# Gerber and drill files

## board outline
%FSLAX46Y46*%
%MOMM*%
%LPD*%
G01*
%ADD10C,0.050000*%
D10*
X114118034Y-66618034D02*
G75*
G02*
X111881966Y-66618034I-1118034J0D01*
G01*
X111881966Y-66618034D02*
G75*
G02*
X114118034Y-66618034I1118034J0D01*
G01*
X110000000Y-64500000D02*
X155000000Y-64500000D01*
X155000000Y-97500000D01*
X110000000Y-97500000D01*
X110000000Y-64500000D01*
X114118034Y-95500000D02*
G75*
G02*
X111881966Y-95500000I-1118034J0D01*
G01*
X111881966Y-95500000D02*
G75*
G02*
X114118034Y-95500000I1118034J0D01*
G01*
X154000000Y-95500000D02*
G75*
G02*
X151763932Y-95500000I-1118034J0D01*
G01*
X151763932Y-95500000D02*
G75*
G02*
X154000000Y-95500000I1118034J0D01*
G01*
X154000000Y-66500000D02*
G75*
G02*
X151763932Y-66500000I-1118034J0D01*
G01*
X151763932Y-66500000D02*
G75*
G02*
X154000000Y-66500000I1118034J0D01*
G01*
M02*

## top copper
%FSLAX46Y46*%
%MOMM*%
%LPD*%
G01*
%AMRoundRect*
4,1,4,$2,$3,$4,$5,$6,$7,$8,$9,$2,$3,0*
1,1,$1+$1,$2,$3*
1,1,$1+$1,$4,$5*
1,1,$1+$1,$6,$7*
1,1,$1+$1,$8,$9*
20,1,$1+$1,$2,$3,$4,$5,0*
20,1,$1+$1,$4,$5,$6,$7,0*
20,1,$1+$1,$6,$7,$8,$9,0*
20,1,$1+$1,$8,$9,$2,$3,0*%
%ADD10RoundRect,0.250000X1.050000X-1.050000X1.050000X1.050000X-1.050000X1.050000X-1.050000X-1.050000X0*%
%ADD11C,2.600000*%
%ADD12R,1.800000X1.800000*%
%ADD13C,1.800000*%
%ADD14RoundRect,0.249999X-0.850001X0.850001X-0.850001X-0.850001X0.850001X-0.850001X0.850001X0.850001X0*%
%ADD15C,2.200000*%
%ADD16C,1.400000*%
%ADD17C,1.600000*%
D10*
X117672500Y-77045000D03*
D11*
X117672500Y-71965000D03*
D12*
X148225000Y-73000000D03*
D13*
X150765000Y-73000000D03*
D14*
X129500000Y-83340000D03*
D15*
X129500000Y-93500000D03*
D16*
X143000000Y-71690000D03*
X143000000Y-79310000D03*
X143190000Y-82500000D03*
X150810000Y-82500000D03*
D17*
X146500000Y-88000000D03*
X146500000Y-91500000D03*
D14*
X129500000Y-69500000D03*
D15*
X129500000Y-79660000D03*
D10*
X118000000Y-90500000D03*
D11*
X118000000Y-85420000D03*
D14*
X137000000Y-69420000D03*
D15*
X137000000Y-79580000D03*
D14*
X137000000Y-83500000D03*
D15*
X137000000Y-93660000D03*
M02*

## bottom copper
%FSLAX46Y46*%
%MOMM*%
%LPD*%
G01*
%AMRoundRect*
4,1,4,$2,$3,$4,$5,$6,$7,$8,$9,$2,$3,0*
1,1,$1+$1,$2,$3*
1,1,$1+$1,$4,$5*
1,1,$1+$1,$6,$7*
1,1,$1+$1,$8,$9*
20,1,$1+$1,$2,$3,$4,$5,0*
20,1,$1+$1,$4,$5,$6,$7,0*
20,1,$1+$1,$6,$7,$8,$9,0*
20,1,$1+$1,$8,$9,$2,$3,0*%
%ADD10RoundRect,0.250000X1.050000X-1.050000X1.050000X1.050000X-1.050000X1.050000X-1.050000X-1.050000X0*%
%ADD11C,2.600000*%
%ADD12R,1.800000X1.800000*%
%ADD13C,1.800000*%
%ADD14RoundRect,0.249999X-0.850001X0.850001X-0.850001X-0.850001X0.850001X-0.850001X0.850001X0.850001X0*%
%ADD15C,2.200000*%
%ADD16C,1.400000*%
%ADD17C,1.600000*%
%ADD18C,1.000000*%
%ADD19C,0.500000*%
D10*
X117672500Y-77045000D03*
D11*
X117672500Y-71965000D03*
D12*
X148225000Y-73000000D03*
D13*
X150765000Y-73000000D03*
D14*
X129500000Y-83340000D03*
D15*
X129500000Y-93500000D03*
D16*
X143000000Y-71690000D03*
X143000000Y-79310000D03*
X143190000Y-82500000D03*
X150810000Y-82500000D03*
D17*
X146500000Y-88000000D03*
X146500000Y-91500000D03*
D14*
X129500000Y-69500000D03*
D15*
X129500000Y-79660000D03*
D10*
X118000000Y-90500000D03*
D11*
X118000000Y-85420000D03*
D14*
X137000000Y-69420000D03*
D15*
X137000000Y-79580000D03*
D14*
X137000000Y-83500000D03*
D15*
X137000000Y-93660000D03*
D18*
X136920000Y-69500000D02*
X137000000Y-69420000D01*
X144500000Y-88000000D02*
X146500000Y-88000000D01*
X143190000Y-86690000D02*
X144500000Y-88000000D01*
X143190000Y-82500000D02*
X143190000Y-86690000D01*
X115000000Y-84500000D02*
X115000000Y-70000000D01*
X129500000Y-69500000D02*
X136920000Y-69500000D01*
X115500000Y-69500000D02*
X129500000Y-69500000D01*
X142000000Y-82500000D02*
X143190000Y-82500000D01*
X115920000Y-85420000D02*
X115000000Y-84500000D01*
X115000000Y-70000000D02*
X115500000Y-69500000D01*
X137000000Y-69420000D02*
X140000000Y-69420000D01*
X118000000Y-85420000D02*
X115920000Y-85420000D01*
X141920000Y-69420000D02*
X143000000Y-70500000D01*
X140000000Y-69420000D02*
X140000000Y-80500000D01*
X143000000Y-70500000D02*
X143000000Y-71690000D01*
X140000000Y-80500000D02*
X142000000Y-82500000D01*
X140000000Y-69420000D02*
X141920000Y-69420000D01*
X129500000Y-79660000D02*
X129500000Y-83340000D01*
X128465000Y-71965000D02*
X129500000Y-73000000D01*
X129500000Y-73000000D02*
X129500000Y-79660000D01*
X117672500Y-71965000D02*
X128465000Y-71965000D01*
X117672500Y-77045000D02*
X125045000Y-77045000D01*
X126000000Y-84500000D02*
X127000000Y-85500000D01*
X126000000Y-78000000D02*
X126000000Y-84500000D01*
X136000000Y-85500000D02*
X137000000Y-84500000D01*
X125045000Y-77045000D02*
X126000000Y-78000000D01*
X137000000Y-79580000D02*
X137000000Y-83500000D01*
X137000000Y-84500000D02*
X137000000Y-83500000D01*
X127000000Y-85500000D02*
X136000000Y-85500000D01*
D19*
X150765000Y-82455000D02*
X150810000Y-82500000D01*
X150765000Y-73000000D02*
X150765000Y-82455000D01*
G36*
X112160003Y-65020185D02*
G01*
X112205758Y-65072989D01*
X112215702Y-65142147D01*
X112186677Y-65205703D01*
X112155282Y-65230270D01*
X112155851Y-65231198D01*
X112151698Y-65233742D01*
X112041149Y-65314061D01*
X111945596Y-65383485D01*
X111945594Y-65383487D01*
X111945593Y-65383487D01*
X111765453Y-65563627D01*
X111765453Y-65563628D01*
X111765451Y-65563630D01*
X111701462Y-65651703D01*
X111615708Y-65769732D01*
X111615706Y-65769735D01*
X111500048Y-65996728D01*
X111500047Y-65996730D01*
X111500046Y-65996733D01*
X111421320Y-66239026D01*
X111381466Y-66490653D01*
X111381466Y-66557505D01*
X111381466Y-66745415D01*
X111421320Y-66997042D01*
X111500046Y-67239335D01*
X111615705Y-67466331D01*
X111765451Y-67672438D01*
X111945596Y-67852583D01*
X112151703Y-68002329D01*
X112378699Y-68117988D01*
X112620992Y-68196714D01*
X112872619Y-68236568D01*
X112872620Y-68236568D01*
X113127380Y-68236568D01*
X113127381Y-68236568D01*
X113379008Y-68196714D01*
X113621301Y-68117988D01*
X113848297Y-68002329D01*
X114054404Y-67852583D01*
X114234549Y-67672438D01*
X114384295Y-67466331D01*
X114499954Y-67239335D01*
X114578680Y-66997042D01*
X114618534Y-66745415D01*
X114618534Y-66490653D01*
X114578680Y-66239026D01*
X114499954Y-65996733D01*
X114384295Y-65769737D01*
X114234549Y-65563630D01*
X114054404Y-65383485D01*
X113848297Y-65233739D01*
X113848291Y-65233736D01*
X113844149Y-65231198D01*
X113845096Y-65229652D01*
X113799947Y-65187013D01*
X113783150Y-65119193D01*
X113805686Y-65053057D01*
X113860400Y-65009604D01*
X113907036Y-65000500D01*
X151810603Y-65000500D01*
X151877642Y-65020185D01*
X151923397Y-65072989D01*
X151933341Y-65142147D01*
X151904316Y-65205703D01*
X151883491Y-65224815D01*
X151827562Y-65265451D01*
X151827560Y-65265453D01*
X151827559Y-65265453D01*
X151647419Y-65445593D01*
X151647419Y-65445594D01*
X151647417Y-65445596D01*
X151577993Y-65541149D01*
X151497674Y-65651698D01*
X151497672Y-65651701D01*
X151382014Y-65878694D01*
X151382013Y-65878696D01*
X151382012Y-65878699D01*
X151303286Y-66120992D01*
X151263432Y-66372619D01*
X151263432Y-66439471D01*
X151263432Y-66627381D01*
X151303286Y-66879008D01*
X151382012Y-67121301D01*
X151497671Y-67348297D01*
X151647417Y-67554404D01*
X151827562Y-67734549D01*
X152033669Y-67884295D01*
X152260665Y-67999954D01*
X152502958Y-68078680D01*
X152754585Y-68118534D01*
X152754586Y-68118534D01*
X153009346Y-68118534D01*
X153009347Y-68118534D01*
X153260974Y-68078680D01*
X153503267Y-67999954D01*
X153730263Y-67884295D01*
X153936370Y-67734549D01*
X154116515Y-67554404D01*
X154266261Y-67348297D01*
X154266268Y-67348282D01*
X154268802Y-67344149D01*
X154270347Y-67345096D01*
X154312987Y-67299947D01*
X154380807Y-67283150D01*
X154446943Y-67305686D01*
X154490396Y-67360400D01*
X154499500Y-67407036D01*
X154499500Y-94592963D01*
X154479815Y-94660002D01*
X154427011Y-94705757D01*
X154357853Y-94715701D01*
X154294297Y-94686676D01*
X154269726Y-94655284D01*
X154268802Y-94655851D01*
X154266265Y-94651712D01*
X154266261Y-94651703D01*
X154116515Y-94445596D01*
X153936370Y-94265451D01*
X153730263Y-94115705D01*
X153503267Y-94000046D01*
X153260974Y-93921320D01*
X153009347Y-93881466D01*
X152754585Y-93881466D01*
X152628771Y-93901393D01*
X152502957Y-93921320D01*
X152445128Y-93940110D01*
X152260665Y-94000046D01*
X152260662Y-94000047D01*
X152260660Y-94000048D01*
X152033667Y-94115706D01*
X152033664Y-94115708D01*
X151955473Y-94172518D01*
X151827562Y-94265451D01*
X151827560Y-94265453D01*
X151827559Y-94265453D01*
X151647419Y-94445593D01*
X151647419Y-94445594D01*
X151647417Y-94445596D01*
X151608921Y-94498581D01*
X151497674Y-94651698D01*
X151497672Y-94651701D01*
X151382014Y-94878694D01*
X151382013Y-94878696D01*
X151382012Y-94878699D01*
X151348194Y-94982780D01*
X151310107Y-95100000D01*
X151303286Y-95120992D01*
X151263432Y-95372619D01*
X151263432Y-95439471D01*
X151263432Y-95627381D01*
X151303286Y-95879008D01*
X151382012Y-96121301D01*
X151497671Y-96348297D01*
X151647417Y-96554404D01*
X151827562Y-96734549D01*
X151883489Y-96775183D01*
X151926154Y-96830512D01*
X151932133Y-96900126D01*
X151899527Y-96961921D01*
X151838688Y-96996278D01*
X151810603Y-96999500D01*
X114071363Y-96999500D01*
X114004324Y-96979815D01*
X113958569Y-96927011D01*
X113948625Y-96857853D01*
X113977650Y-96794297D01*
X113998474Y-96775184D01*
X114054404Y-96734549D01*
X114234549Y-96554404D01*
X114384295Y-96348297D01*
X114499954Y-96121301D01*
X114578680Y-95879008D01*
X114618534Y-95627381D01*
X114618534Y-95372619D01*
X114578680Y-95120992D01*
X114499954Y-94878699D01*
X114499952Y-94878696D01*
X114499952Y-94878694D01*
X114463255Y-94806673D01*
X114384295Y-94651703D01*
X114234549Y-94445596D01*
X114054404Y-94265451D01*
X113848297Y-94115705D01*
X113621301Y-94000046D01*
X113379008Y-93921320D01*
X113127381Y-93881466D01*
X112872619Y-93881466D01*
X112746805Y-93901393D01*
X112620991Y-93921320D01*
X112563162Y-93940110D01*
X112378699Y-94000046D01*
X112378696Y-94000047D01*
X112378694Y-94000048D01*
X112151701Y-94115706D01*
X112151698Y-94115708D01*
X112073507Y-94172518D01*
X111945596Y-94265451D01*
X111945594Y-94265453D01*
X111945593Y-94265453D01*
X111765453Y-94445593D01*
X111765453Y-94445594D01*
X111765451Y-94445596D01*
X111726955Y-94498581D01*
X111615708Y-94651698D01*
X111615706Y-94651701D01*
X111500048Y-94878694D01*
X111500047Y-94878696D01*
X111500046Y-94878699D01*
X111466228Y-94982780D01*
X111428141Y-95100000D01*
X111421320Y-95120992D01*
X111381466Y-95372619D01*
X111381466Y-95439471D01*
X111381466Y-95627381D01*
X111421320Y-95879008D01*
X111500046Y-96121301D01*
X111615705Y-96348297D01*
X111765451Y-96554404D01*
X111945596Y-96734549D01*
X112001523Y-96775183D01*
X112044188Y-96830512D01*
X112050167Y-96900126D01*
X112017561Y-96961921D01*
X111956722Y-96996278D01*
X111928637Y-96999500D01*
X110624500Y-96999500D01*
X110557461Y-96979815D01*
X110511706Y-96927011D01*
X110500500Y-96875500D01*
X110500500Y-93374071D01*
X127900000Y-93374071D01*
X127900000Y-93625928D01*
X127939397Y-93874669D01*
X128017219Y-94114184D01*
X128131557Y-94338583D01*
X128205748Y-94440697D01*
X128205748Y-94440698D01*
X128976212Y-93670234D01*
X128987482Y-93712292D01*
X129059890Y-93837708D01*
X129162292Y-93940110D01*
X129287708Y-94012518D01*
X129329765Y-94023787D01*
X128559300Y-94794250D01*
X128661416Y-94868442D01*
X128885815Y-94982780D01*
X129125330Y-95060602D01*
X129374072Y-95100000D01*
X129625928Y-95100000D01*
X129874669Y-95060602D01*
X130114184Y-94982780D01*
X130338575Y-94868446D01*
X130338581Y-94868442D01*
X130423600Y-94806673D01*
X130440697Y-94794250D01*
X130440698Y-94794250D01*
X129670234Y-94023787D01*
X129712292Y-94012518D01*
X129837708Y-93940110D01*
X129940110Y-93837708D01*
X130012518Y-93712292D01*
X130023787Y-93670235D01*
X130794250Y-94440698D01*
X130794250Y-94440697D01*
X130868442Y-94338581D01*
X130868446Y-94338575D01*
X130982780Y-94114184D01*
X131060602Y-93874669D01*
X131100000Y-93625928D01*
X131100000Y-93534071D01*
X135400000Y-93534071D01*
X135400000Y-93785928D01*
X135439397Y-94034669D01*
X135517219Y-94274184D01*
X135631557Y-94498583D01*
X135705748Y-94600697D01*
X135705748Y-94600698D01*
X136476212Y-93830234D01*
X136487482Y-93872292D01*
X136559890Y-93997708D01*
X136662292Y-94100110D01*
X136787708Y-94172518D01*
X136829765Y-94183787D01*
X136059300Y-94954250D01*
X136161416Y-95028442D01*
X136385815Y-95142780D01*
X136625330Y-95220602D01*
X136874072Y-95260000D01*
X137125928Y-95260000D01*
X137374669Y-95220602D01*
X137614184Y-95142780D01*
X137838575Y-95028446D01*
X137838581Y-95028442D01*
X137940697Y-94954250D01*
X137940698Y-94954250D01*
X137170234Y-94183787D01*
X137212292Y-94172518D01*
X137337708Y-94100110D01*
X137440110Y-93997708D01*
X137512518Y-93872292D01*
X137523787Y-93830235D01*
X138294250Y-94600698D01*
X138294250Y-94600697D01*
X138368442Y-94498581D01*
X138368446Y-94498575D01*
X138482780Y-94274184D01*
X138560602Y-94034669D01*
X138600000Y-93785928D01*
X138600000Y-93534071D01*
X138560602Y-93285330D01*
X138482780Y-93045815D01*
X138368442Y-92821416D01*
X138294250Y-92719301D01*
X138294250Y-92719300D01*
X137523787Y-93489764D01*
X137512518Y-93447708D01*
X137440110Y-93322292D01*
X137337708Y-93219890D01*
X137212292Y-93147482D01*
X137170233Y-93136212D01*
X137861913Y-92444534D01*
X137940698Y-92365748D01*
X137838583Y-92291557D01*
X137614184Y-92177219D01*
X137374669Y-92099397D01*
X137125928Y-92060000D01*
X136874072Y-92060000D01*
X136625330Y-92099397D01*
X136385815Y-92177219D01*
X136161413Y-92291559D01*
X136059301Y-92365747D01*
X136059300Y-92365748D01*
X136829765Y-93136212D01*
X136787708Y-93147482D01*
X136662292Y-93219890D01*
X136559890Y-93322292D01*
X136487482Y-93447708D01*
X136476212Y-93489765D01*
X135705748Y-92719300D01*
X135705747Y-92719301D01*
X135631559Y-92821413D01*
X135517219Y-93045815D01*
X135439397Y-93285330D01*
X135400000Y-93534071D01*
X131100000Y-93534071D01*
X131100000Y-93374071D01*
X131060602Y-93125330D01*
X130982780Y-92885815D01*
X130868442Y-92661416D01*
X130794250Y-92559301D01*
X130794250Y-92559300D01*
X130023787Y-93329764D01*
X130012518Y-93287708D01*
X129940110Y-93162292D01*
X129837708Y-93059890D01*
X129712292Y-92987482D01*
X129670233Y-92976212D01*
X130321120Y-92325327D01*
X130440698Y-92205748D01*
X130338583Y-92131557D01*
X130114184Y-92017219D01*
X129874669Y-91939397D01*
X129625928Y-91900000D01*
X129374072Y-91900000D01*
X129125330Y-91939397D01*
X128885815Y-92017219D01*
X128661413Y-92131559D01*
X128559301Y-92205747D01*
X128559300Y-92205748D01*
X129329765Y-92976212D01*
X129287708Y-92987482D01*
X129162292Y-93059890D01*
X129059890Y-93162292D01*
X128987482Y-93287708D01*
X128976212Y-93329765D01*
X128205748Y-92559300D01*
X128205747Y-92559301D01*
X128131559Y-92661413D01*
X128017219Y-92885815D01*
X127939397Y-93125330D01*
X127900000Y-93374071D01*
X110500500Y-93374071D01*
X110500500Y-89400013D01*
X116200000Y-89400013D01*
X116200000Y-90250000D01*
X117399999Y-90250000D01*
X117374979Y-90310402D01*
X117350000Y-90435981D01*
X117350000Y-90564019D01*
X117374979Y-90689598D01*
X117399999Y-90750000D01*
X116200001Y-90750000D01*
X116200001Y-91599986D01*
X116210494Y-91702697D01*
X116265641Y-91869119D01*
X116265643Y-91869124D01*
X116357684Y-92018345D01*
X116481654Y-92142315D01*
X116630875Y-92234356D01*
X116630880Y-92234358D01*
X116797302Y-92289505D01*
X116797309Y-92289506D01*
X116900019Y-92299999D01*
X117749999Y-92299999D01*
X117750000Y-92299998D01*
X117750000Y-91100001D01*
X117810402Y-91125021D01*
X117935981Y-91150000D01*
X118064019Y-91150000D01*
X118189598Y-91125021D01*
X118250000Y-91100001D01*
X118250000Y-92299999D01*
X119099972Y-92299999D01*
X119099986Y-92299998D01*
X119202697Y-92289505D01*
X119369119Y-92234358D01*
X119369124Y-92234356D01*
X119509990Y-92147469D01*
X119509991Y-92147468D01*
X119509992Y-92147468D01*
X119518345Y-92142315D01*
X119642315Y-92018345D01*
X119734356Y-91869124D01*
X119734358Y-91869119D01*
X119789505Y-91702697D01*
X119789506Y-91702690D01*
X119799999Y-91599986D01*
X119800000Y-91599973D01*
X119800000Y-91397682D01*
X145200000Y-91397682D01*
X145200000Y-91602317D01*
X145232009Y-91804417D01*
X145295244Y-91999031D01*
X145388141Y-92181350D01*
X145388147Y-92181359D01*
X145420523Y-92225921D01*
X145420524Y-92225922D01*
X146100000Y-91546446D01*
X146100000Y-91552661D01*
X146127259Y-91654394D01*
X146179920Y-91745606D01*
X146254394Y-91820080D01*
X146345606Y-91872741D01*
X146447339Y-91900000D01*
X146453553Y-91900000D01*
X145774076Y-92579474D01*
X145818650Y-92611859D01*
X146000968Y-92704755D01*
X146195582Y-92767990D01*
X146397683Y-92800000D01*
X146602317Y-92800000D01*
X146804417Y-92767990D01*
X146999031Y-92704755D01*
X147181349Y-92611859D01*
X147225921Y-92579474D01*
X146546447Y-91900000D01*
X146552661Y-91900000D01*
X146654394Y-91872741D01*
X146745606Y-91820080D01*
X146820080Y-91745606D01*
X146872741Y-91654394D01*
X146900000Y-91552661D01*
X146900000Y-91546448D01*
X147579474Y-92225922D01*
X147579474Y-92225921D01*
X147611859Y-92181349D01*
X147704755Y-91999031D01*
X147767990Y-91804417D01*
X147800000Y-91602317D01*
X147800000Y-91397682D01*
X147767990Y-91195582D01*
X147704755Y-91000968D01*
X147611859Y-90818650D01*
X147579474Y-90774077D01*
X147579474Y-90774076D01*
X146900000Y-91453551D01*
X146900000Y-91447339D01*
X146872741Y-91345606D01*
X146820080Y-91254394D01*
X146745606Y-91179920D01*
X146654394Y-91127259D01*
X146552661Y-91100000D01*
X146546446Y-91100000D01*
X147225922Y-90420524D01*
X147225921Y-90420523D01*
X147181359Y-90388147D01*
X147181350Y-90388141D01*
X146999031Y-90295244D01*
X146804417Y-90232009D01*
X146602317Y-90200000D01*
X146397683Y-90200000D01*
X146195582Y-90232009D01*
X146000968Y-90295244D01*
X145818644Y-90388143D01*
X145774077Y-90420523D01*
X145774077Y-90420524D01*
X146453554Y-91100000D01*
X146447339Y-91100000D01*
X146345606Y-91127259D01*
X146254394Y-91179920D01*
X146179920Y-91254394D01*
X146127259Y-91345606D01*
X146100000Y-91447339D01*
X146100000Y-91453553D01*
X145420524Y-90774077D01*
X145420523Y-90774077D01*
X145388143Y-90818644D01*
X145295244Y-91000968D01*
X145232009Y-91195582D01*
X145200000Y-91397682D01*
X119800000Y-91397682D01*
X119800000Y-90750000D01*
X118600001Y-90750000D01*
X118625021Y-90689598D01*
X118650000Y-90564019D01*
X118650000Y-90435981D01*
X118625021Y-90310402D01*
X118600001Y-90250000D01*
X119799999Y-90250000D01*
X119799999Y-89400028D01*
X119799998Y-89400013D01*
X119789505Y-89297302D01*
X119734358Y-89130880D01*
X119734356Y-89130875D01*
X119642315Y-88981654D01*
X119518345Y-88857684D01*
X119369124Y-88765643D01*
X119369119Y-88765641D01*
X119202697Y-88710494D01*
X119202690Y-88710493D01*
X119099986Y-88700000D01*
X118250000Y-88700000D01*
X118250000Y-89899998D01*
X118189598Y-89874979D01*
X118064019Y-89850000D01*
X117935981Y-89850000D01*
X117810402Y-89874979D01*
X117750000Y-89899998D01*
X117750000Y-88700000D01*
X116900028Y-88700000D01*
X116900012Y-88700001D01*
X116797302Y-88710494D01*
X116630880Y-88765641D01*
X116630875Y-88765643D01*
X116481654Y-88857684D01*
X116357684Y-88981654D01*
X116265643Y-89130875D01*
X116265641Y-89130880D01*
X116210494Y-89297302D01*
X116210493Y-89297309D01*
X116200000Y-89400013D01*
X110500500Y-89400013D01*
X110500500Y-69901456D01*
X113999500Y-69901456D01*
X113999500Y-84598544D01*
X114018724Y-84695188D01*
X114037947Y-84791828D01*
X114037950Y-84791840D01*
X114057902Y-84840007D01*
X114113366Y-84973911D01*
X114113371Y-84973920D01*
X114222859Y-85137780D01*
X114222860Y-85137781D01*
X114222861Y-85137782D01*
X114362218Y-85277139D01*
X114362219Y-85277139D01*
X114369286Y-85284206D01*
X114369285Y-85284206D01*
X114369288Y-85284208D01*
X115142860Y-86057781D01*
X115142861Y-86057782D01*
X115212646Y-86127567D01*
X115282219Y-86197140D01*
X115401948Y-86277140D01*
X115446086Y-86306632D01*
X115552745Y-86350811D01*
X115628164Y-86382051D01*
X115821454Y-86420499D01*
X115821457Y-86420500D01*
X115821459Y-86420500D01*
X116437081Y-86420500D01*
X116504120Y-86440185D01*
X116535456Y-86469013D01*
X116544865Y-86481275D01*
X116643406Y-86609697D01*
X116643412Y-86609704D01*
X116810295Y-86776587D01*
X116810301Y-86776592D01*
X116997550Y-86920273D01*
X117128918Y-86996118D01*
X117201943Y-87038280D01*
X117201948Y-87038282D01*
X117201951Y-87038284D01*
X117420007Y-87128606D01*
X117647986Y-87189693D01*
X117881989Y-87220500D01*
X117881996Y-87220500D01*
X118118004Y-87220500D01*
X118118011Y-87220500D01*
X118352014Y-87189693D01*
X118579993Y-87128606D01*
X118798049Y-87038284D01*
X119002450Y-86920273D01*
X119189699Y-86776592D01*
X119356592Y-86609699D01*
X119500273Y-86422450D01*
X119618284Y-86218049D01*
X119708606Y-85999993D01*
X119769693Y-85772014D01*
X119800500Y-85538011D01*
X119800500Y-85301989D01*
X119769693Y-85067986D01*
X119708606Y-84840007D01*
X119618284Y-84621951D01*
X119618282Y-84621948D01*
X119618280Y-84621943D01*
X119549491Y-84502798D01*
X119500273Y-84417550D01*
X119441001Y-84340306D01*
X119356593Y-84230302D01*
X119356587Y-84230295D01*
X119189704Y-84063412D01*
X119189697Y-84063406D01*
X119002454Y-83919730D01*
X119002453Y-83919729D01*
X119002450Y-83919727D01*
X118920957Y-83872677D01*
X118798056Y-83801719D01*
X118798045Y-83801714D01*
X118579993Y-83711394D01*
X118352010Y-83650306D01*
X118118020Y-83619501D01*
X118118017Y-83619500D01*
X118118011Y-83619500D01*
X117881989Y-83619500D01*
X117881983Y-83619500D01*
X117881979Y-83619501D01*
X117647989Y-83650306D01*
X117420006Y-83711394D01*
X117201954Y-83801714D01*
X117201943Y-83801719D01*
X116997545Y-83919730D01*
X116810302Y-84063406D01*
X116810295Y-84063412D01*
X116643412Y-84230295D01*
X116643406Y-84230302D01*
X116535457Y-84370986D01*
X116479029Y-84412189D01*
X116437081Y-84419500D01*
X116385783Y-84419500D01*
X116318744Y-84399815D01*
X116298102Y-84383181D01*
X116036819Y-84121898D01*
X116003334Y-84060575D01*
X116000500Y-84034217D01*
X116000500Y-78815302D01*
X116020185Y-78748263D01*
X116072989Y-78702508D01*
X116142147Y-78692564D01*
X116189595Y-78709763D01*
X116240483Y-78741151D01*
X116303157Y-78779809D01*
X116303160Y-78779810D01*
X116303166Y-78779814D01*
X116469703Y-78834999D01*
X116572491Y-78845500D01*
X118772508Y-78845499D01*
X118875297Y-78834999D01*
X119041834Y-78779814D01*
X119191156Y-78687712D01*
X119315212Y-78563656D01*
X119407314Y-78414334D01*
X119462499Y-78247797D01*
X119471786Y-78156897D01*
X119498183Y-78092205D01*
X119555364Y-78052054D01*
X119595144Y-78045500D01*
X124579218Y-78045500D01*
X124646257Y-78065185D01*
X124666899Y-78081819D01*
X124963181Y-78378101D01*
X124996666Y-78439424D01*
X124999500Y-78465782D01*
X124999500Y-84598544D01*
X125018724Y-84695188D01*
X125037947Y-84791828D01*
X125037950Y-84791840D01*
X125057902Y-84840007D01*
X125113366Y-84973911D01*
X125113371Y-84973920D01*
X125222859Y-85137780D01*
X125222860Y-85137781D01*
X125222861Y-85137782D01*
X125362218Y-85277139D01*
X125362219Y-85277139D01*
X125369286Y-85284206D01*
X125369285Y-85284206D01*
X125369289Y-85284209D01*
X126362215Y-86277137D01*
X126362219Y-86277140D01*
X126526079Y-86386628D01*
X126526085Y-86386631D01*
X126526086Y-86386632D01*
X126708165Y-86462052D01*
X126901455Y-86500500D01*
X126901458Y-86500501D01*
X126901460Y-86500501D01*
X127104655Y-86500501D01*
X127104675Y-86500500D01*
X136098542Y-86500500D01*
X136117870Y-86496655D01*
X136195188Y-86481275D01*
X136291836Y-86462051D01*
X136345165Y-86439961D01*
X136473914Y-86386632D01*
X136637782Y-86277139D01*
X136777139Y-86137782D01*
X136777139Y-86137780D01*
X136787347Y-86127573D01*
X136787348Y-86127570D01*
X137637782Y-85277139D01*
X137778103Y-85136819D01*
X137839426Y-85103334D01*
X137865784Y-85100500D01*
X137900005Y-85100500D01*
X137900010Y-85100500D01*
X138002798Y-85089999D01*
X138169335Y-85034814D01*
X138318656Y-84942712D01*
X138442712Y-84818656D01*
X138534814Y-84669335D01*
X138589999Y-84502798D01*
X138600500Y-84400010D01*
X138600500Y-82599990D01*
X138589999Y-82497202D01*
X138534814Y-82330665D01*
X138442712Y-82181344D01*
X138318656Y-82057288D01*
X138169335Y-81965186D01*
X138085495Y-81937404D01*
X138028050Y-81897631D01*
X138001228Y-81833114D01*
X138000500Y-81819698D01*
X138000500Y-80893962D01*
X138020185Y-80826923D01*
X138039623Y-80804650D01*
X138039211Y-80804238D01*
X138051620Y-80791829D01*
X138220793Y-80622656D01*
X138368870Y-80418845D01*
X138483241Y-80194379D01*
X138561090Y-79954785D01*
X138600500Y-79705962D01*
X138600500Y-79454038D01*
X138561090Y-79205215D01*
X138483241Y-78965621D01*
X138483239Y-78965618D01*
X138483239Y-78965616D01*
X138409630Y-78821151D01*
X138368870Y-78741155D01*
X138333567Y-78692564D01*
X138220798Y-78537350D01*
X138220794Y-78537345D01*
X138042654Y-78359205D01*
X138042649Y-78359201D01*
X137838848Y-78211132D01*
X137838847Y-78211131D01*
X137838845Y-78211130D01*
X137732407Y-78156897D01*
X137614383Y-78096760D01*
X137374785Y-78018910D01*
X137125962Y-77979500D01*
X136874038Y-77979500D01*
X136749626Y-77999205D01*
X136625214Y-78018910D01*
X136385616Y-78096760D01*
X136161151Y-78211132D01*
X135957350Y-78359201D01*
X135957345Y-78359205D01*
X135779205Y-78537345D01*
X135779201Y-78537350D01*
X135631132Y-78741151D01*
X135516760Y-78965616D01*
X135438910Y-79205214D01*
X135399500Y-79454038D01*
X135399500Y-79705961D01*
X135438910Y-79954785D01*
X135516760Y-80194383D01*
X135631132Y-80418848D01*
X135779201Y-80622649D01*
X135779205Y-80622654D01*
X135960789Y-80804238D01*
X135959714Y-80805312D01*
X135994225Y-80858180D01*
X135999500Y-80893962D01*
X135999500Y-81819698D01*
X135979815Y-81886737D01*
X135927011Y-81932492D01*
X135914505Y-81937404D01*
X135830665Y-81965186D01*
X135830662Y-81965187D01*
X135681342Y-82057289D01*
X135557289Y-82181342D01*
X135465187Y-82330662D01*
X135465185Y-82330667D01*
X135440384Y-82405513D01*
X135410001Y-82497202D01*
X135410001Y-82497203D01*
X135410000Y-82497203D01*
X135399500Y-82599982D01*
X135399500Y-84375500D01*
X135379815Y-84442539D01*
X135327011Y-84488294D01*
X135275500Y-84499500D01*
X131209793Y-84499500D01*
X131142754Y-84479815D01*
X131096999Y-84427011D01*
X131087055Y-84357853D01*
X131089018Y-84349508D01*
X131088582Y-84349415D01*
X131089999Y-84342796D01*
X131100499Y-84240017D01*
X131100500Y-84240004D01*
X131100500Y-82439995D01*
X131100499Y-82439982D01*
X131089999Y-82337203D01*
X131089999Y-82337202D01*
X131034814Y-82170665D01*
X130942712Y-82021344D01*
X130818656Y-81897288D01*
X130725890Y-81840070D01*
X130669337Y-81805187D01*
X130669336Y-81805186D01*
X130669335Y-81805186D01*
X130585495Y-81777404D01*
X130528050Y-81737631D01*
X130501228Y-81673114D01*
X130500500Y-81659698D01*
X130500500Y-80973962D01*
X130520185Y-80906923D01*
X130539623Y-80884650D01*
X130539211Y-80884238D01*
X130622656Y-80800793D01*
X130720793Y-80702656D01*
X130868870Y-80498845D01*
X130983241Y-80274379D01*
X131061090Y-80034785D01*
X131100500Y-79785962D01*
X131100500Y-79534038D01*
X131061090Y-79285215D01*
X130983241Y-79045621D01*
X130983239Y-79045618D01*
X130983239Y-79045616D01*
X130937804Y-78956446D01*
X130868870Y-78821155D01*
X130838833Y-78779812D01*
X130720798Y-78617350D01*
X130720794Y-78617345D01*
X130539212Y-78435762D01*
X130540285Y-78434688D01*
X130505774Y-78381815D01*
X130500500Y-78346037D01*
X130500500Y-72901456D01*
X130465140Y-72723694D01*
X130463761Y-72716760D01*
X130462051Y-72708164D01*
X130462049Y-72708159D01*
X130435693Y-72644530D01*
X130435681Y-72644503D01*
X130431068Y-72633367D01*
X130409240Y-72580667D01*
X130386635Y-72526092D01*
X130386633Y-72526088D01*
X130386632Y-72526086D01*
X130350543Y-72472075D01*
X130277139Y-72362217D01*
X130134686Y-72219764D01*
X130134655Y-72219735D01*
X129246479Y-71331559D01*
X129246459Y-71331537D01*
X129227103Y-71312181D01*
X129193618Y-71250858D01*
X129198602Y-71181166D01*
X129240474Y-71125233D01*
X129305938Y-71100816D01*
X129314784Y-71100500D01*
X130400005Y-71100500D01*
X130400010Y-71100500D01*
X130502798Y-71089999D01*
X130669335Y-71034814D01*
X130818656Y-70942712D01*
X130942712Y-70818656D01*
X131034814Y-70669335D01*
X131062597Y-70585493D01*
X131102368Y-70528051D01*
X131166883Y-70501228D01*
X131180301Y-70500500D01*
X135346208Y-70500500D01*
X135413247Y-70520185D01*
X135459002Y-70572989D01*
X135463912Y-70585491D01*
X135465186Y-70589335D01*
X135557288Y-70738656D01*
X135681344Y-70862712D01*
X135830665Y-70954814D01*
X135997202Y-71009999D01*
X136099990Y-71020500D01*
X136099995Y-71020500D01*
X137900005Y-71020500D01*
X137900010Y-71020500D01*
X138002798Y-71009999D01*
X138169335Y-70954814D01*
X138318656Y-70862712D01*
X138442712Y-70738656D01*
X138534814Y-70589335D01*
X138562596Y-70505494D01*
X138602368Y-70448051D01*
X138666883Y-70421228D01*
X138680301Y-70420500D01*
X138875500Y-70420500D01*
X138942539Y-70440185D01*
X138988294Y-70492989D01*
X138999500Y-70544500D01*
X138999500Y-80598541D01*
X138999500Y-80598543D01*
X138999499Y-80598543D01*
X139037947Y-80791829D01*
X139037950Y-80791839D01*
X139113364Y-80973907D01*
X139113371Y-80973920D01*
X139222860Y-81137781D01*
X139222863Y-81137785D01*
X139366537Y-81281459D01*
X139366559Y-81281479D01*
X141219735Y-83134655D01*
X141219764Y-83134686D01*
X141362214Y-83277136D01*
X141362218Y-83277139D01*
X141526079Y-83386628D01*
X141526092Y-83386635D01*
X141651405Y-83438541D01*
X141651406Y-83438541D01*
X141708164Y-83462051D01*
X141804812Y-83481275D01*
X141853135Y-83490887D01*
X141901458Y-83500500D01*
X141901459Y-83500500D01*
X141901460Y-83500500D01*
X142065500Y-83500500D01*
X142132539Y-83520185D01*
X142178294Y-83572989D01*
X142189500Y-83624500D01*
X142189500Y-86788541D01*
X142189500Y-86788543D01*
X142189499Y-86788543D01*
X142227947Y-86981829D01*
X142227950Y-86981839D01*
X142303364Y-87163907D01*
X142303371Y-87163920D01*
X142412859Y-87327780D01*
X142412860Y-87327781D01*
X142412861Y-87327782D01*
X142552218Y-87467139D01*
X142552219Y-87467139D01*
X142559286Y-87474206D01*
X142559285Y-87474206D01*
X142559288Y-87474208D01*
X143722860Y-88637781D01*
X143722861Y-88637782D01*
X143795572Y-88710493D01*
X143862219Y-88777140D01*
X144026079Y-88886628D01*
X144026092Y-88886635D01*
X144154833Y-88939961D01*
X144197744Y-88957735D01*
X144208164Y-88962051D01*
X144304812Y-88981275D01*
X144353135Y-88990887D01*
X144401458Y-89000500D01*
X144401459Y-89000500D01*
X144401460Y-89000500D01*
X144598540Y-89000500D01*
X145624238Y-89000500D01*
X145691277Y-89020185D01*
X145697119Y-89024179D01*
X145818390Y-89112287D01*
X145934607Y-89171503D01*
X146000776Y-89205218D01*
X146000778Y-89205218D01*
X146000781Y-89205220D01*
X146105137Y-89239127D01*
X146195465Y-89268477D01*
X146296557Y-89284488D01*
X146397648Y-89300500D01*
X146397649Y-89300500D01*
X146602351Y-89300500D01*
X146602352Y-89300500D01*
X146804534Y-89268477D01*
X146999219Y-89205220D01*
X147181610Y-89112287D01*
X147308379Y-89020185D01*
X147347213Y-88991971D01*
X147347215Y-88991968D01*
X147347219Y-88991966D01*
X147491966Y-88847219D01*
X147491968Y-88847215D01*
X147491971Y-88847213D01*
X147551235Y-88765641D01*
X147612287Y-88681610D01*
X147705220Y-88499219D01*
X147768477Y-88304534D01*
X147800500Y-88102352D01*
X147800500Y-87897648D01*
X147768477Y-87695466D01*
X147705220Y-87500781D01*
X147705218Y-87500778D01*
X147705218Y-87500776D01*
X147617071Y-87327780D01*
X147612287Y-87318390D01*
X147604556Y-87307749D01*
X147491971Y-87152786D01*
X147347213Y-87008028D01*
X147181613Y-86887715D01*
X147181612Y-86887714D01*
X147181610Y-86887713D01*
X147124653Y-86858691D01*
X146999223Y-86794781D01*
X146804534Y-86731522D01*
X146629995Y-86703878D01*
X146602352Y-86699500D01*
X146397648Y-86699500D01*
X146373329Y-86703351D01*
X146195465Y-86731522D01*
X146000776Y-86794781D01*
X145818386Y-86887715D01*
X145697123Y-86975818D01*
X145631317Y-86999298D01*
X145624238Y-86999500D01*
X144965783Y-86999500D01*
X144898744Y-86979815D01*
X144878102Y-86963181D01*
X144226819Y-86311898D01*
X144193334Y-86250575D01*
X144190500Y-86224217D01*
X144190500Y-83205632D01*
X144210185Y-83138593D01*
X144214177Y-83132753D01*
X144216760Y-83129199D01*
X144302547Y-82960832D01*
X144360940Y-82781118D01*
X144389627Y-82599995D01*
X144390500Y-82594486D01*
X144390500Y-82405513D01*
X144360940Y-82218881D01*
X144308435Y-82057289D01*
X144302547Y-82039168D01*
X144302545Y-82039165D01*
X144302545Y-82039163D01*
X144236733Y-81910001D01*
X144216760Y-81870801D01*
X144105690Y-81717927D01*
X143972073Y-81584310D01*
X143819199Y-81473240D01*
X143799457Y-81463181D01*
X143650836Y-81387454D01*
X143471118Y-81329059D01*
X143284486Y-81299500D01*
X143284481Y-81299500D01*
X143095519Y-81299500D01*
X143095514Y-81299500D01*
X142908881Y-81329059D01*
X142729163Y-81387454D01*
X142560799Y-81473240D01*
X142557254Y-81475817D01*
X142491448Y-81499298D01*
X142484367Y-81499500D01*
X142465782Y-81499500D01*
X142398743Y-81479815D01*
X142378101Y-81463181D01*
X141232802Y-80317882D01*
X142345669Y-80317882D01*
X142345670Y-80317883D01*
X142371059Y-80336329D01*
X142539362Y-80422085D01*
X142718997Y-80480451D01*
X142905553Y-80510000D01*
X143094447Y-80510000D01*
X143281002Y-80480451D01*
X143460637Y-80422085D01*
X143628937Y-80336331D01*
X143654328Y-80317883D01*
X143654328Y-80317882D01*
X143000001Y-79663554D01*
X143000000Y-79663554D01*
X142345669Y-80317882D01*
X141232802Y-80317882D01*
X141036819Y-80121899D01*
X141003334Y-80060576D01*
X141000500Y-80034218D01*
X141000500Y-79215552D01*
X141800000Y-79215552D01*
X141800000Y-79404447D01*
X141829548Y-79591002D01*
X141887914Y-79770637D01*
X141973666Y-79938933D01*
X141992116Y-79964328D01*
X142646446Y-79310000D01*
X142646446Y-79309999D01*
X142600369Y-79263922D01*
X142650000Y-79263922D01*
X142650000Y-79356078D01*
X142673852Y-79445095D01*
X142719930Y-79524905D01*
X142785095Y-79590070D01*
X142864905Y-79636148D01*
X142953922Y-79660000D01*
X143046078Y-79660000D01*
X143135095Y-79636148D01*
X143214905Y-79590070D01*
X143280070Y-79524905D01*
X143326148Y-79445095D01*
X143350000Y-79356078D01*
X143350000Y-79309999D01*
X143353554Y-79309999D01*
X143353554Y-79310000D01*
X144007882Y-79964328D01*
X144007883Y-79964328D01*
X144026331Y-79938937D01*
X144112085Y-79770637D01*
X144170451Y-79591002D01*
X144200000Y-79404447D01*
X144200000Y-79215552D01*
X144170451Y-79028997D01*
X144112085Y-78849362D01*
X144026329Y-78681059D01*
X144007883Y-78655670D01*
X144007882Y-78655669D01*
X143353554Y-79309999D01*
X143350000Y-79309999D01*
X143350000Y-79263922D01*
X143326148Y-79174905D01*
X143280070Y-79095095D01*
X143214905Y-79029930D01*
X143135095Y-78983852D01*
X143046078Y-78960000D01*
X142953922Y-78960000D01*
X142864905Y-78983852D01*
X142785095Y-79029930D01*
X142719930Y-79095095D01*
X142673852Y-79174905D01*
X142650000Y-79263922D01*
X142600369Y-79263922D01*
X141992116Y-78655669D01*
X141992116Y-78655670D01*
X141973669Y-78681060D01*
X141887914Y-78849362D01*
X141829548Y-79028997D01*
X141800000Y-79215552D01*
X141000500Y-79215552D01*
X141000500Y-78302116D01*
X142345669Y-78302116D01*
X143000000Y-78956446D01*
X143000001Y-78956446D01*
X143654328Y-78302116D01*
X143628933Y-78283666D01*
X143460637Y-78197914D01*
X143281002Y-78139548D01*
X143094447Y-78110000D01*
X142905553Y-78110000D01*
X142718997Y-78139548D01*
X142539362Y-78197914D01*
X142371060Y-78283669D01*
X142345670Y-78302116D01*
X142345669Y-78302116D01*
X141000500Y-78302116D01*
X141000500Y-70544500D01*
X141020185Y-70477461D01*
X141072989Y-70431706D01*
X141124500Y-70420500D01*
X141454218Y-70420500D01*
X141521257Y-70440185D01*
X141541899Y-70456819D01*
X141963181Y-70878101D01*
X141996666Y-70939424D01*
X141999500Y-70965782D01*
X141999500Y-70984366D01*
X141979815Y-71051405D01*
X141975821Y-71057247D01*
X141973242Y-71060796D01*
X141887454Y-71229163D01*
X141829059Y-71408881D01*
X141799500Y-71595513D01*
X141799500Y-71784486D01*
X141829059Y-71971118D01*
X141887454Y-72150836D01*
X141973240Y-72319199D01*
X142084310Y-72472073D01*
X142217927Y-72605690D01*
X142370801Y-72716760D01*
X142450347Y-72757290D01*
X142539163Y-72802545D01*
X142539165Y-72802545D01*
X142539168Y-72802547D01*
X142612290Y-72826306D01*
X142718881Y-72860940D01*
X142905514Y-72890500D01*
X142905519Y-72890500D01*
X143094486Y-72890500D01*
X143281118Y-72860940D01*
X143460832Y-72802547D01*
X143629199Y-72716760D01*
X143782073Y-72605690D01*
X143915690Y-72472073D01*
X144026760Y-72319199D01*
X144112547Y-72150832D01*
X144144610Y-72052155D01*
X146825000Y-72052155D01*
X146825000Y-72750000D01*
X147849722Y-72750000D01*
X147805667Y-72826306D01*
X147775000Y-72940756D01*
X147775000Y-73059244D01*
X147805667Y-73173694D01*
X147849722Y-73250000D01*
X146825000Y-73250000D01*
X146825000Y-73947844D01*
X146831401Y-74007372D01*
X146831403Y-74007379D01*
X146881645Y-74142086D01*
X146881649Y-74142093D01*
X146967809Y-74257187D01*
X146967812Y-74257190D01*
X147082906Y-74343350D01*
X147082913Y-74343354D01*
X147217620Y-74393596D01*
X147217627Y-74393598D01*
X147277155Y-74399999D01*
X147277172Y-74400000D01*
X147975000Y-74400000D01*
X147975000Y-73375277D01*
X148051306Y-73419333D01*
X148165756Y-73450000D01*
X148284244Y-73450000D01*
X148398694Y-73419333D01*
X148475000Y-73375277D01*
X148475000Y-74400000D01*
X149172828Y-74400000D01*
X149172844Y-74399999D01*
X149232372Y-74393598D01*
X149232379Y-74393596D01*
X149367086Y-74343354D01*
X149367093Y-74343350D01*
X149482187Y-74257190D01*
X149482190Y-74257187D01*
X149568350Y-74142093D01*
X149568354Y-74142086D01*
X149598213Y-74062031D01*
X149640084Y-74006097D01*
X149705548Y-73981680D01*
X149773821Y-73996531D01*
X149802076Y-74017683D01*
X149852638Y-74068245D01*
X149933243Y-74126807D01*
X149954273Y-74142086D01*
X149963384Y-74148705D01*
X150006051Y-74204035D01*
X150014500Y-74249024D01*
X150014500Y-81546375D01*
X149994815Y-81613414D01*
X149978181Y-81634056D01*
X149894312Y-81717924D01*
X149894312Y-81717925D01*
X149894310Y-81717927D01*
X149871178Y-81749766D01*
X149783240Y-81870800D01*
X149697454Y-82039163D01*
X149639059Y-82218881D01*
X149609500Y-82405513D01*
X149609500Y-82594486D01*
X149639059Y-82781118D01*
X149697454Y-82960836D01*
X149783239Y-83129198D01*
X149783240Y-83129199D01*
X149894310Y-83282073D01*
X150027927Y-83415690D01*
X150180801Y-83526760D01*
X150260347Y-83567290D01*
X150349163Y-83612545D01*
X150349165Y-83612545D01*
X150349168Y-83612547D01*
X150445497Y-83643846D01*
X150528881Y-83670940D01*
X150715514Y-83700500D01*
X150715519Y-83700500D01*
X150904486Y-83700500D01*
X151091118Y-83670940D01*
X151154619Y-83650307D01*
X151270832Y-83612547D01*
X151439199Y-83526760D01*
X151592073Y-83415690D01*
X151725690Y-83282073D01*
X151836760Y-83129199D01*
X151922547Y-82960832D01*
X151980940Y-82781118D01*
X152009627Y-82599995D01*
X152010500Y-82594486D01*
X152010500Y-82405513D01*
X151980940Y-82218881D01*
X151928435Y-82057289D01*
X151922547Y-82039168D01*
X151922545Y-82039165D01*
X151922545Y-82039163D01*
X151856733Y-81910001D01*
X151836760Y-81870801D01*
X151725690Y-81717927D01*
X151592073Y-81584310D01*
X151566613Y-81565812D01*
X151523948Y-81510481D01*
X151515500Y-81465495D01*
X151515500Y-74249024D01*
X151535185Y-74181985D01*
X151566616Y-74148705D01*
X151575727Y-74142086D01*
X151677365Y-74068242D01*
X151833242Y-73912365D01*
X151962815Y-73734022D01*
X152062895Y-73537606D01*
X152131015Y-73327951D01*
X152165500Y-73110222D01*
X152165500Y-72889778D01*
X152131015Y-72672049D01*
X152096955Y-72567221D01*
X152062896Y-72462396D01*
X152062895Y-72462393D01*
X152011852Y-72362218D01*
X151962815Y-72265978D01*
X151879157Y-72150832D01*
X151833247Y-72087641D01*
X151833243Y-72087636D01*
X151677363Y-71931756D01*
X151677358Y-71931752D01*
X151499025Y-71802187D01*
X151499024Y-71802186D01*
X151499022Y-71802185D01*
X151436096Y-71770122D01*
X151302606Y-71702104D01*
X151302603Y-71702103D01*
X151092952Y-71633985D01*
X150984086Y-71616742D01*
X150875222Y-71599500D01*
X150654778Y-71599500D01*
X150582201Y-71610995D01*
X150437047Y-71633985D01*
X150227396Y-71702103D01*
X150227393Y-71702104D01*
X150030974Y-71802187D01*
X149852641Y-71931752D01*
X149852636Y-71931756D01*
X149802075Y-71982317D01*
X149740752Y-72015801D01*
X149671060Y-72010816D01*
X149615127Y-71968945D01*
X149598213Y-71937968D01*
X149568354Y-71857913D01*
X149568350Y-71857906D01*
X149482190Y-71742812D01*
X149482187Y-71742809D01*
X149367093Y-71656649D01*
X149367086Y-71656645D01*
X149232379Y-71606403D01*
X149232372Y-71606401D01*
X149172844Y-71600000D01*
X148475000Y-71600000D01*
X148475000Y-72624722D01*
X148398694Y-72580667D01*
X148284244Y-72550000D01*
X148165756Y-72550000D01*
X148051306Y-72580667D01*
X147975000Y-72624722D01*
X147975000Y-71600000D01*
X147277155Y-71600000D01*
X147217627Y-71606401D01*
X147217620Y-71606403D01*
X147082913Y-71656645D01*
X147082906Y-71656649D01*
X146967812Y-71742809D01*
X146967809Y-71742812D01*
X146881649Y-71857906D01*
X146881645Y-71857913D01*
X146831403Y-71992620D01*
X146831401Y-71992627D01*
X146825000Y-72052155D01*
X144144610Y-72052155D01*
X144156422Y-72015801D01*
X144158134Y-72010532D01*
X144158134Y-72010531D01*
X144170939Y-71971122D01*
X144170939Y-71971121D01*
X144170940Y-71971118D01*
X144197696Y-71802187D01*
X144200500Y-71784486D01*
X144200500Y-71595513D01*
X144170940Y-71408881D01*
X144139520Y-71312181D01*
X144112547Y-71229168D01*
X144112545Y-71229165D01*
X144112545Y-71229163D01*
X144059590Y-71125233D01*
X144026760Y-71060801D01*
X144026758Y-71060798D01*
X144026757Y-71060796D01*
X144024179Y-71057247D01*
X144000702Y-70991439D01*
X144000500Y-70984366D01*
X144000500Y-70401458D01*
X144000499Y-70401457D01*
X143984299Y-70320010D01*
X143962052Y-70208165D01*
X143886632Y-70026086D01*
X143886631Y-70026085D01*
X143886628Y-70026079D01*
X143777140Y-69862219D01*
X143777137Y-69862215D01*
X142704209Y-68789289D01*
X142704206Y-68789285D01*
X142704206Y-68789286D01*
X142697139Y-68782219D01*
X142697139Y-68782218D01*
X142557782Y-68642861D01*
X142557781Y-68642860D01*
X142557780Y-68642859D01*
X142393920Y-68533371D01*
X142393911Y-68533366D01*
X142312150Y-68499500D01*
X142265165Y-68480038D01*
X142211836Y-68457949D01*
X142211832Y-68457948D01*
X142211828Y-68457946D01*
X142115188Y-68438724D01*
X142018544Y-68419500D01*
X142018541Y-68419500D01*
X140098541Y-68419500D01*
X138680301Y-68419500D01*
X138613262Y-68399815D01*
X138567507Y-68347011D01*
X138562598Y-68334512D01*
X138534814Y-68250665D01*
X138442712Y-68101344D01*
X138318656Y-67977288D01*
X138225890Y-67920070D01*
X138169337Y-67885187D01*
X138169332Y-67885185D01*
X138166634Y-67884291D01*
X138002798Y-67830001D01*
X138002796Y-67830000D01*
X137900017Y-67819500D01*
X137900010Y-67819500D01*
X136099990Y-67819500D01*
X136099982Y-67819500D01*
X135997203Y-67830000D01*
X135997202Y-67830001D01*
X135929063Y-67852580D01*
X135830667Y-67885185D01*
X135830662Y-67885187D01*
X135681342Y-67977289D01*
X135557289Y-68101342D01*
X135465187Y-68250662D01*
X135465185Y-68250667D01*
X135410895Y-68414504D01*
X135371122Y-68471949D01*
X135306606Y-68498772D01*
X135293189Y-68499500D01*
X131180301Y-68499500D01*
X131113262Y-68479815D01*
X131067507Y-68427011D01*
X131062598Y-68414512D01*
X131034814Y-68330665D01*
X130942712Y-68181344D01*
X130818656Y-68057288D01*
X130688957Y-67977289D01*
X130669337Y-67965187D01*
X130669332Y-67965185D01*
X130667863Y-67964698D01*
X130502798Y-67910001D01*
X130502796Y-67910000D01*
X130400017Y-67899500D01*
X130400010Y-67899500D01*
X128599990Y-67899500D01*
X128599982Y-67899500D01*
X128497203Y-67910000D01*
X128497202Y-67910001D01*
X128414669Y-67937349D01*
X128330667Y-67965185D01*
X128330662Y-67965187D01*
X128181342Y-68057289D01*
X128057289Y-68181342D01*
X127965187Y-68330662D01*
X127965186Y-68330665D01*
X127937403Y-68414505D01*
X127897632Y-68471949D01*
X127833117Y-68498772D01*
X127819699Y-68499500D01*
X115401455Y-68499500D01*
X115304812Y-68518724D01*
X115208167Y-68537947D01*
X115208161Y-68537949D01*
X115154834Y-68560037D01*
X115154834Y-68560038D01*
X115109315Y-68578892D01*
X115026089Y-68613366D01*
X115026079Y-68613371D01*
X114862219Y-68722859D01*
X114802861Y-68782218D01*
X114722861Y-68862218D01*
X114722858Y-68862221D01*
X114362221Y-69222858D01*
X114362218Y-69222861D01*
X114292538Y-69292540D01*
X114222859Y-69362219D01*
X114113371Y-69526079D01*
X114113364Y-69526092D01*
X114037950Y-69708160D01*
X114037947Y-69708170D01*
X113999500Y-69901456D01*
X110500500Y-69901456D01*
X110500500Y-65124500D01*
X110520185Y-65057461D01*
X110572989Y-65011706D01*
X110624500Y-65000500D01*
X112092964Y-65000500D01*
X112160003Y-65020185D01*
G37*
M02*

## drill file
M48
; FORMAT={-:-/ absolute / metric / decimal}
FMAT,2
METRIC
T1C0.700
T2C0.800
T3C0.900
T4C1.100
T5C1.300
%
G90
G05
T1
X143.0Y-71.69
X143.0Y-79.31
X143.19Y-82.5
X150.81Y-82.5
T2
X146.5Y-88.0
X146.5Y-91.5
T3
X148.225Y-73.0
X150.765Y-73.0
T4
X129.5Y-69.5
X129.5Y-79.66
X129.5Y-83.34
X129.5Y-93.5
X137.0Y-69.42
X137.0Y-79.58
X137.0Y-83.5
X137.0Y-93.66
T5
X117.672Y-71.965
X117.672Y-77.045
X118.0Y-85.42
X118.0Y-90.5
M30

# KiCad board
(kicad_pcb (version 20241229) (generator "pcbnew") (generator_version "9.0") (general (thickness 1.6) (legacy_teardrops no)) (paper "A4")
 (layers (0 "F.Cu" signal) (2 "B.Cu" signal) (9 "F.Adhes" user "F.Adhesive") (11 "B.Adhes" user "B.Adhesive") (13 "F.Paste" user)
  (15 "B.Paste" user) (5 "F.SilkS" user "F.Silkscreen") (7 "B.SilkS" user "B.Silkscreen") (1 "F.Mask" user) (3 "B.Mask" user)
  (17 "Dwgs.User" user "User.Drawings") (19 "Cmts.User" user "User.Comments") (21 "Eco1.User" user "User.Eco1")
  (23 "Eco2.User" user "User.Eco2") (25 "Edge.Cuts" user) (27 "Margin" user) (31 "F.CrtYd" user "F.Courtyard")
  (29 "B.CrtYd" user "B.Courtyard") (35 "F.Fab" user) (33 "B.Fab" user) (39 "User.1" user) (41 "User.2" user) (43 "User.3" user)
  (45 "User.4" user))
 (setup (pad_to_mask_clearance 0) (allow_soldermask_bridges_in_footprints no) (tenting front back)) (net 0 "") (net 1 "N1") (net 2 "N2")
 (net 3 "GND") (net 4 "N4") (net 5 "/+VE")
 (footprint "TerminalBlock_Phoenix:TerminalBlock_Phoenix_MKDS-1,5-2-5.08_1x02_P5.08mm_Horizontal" (layer "F.Cu") (at 117.6725 77.045 90)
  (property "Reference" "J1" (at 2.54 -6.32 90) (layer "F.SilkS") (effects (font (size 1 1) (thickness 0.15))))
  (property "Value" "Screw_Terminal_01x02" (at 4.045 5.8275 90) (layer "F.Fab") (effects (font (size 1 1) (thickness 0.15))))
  (pad "1" thru_hole roundrect (at 0 0 90) (size 2.6 2.6) (drill 1.3) (layers "*.Cu" "*.Mask") (remove_unused_layers no)
   (roundrect_rratio 0.096154) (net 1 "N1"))
  (pad "2" thru_hole circle (at 5.08 0 90) (size 2.6 2.6) (drill 1.3) (layers "*.Cu" "*.Mask") (remove_unused_layers no) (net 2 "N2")))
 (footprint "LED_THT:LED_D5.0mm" (layer "F.Cu") (at 148.225 73)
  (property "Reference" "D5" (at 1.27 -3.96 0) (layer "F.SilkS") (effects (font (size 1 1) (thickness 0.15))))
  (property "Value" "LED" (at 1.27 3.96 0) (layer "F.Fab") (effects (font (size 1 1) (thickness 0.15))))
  (pad "1" thru_hole rect (at 0 0) (size 1.8 1.8) (drill 0.9) (layers "*.Cu" "*.Mask") (remove_unused_layers no) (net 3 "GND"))
  (pad "2" thru_hole circle (at 2.54 0) (size 1.8 1.8) (drill 0.9) (layers "*.Cu" "*.Mask") (remove_unused_layers no) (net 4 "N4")))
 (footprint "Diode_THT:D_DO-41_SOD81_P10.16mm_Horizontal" (layer "F.Cu") (at 129.5 83.34 -90)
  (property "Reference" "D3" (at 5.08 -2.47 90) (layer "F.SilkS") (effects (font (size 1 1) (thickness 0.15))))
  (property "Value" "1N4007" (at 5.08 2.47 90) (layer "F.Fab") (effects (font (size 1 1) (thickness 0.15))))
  (pad "1" thru_hole roundrect (at 0 0 270) (size 2.2 2.2) (drill 1.1) (layers "*.Cu" "*.Mask") (remove_unused_layers no)
   (roundrect_rratio 0.113636) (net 2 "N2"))
  (pad "2" thru_hole circle (at 10.16 0 270) (size 2.2 2.2) (drill 1.1) (layers "*.Cu" "*.Mask") (remove_unused_layers no) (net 3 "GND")))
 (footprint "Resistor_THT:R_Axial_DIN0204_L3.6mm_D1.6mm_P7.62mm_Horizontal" (layer "F.Cu") (at 143 71.69 -90)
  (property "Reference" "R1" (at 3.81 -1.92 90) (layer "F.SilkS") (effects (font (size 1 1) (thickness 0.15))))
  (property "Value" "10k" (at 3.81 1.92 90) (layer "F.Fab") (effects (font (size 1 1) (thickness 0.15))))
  (pad "1" thru_hole circle (at 0 0 270) (size 1.4 1.4) (drill 0.7) (layers "*.Cu" "*.Mask") (remove_unused_layers no) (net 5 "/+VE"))
  (pad "2" thru_hole circle (at 7.62 0 270) (size 1.4 1.4) (drill 0.7) (layers "*.Cu" "*.Mask") (remove_unused_layers no) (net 3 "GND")))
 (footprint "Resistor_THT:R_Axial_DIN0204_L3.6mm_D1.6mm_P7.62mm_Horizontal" (layer "F.Cu") (at 143.19 82.5)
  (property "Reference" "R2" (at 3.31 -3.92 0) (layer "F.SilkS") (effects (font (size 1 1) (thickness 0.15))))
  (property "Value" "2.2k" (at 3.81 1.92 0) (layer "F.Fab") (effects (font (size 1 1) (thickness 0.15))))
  (pad "1" thru_hole circle (at 0 0) (size 1.4 1.4) (drill 0.7) (layers "*.Cu" "*.Mask") (remove_unused_layers no) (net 5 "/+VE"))
  (pad "2" thru_hole circle (at 7.62 0) (size 1.4 1.4) (drill 0.7) (layers "*.Cu" "*.Mask") (remove_unused_layers no) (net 4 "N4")))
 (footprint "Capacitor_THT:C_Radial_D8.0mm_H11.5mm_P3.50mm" (layer "F.Cu") (at 146.5 88 -90)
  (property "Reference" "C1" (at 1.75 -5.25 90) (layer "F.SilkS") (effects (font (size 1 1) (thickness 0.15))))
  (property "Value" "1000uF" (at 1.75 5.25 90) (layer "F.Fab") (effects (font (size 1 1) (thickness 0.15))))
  (pad "1" thru_hole circle (at 0 0 270) (size 1.6 1.6) (drill 0.8) (layers "*.Cu" "*.Mask") (remove_unused_layers no) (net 5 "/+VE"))
  (pad "2" thru_hole circle (at 3.5 0 270) (size 1.6 1.6) (drill 0.8) (layers "*.Cu" "*.Mask") (remove_unused_layers no) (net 3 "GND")))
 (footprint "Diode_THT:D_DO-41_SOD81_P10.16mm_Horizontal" (layer "F.Cu") (at 129.5 69.5 -90)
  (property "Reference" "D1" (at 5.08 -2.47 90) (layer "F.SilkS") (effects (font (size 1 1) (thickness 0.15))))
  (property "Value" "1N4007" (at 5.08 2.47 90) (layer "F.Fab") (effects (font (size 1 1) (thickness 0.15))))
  (pad "1" thru_hole roundrect (at 0 0 270) (size 2.2 2.2) (drill 1.1) (layers "*.Cu" "*.Mask") (remove_unused_layers no)
   (roundrect_rratio 0.113636) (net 5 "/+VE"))
  (pad "2" thru_hole circle (at 10.16 0 270) (size 2.2 2.2) (drill 1.1) (layers "*.Cu" "*.Mask") (remove_unused_layers no) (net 2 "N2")))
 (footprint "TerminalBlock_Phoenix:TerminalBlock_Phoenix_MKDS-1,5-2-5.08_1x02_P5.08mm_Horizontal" (layer "F.Cu") (at 118 90.5 90)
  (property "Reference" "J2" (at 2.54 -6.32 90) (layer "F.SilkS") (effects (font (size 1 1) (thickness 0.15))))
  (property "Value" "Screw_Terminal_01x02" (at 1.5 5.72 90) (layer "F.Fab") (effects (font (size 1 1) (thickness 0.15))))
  (pad "1" thru_hole roundrect (at 0 0 90) (size 2.6 2.6) (drill 1.3) (layers "*.Cu" "*.Mask") (remove_unused_layers no)
   (roundrect_rratio 0.096154) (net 3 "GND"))
  (pad "2" thru_hole circle (at 5.08 0 90) (size 2.6 2.6) (drill 1.3) (layers "*.Cu" "*.Mask") (remove_unused_layers no) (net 5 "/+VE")))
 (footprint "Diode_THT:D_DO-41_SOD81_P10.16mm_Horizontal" (layer "F.Cu") (at 137 69.42 -90)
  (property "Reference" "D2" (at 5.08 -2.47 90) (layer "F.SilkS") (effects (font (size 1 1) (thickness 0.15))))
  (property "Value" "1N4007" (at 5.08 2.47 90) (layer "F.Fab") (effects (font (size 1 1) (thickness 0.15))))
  (pad "1" thru_hole roundrect (at 0 0 270) (size 2.2 2.2) (drill 1.1) (layers "*.Cu" "*.Mask") (remove_unused_layers no)
   (roundrect_rratio 0.113636) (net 5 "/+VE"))
  (pad "2" thru_hole circle (at 10.16 0 270) (size 2.2 2.2) (drill 1.1) (layers "*.Cu" "*.Mask") (remove_unused_layers no) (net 1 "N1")))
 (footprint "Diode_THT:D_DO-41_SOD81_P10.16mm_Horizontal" (layer "F.Cu") (at 137 83.5 -90)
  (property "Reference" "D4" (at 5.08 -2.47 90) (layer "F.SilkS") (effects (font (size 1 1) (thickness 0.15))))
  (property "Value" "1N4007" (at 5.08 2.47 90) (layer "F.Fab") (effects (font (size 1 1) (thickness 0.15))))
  (pad "1" thru_hole roundrect (at 0 0 270) (size 2.2 2.2) (drill 1.1) (layers "*.Cu" "*.Mask") (remove_unused_layers no)
   (roundrect_rratio 0.113636) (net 1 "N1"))
  (pad "2" thru_hole circle (at 10.16 0 270) (size 2.2 2.2) (drill 1.1) (layers "*.Cu" "*.Mask") (remove_unused_layers no) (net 3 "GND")))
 (gr_circle (center 113 66.618034) (end 114 67.118034) (stroke (width 0.05) (type default)) (fill no) (layer "Edge.Cuts"))
 (gr_rect (start 110 64.5) (end 155 97.5) (stroke (width 0.05) (type default)) (fill no) (layer "Edge.Cuts"))
 (gr_circle (center 113 95.5) (end 114 96) (stroke (width 0.05) (type default)) (fill no) (layer "Edge.Cuts"))
 (gr_circle (center 152.881966 95.5) (end 153.881966 96) (stroke (width 0.05) (type default)) (fill no) (layer "Edge.Cuts"))
 (gr_circle (center 152.881966 66.5) (end 153.881966 67) (stroke (width 0.05) (type default)) (fill no) (layer "Edge.Cuts"))
 (segment (start 136.92 69.5) (end 137 69.42) (width 1) (layer "B.Cu") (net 5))
 (segment (start 144.5 88) (end 146.5 88) (width 1) (layer "B.Cu") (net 5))
 (segment (start 143.19 86.69) (end 144.5 88) (width 1) (layer "B.Cu") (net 5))
 (segment (start 143.19 82.5) (end 143.19 86.69) (width 1) (layer "B.Cu") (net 5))
 (segment (start 115 84.5) (end 115 70) (width 1) (layer "B.Cu") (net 5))
 (segment (start 129.5 69.5) (end 136.92 69.5) (width 1) (layer "B.Cu") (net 5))
 (segment (start 115.5 69.5) (end 129.5 69.5) (width 1) (layer "B.Cu") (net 5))
 (segment (start 142 82.5) (end 143.19 82.5) (width 1) (layer "B.Cu") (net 5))
 (segment (start 115.92 85.42) (end 115 84.5) (width 1) (layer "B.Cu") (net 5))
 (segment (start 115 70) (end 115.5 69.5) (width 1) (layer "B.Cu") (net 5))
 (segment (start 137 69.42) (end 140 69.42) (width 1) (layer "B.Cu") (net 5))
 (segment (start 118 85.42) (end 115.92 85.42) (width 1) (layer "B.Cu") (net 5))
 (segment (start 141.92 69.42) (end 143 70.5) (width 1) (layer "B.Cu") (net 5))
 (segment (start 140 69.42) (end 140 80.5) (width 1) (layer "B.Cu") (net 5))
 (segment (start 143 70.5) (end 143 71.69) (width 1) (layer "B.Cu") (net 5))
 (segment (start 140 80.5) (end 142 82.5) (width 1) (layer "B.Cu") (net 5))
 (segment (start 140 69.42) (end 141.92 69.42) (width 1) (layer "B.Cu") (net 5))
 (segment (start 129.5 79.66) (end 129.5 83.34) (width 1) (layer "B.Cu") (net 2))
 (segment (start 128.465 71.965) (end 129.5 73) (width 1) (layer "B.Cu") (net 2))
 (segment (start 129.5 73) (end 129.5 79.66) (width 1) (layer "B.Cu") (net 2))
 (segment (start 117.6725 71.965) (end 128.465 71.965) (width 1) (layer "B.Cu") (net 2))
 (segment (start 117.6725 77.045) (end 125.045 77.045) (width 1) (layer "B.Cu") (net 1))
 (segment (start 126 84.5) (end 127 85.5) (width 1) (layer "B.Cu") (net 1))
 (segment (start 126 78) (end 126 84.5) (width 1) (layer "B.Cu") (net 1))
 (segment (start 136 85.5) (end 137 84.5) (width 1) (layer "B.Cu") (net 1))
 (segment (start 125.045 77.045) (end 126 78) (width 1) (layer "B.Cu") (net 1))
 (segment (start 137 79.58) (end 137 83.5) (width 1) (layer "B.Cu") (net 1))
 (segment (start 137 84.5) (end 137 83.5) (width 1) (layer "B.Cu") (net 1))
 (segment (start 127 85.5) (end 136 85.5) (width 1) (layer "B.Cu") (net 1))
 (segment (start 150.765 82.455) (end 150.81 82.5) (width 0.5) (layer "B.Cu") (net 4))
 (segment (start 150.765 73) (end 150.765 82.455) (width 0.5) (layer "B.Cu") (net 4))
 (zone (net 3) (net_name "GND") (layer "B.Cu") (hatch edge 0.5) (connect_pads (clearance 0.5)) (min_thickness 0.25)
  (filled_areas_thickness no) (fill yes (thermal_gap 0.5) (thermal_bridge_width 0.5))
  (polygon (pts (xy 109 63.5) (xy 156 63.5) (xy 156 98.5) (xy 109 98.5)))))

